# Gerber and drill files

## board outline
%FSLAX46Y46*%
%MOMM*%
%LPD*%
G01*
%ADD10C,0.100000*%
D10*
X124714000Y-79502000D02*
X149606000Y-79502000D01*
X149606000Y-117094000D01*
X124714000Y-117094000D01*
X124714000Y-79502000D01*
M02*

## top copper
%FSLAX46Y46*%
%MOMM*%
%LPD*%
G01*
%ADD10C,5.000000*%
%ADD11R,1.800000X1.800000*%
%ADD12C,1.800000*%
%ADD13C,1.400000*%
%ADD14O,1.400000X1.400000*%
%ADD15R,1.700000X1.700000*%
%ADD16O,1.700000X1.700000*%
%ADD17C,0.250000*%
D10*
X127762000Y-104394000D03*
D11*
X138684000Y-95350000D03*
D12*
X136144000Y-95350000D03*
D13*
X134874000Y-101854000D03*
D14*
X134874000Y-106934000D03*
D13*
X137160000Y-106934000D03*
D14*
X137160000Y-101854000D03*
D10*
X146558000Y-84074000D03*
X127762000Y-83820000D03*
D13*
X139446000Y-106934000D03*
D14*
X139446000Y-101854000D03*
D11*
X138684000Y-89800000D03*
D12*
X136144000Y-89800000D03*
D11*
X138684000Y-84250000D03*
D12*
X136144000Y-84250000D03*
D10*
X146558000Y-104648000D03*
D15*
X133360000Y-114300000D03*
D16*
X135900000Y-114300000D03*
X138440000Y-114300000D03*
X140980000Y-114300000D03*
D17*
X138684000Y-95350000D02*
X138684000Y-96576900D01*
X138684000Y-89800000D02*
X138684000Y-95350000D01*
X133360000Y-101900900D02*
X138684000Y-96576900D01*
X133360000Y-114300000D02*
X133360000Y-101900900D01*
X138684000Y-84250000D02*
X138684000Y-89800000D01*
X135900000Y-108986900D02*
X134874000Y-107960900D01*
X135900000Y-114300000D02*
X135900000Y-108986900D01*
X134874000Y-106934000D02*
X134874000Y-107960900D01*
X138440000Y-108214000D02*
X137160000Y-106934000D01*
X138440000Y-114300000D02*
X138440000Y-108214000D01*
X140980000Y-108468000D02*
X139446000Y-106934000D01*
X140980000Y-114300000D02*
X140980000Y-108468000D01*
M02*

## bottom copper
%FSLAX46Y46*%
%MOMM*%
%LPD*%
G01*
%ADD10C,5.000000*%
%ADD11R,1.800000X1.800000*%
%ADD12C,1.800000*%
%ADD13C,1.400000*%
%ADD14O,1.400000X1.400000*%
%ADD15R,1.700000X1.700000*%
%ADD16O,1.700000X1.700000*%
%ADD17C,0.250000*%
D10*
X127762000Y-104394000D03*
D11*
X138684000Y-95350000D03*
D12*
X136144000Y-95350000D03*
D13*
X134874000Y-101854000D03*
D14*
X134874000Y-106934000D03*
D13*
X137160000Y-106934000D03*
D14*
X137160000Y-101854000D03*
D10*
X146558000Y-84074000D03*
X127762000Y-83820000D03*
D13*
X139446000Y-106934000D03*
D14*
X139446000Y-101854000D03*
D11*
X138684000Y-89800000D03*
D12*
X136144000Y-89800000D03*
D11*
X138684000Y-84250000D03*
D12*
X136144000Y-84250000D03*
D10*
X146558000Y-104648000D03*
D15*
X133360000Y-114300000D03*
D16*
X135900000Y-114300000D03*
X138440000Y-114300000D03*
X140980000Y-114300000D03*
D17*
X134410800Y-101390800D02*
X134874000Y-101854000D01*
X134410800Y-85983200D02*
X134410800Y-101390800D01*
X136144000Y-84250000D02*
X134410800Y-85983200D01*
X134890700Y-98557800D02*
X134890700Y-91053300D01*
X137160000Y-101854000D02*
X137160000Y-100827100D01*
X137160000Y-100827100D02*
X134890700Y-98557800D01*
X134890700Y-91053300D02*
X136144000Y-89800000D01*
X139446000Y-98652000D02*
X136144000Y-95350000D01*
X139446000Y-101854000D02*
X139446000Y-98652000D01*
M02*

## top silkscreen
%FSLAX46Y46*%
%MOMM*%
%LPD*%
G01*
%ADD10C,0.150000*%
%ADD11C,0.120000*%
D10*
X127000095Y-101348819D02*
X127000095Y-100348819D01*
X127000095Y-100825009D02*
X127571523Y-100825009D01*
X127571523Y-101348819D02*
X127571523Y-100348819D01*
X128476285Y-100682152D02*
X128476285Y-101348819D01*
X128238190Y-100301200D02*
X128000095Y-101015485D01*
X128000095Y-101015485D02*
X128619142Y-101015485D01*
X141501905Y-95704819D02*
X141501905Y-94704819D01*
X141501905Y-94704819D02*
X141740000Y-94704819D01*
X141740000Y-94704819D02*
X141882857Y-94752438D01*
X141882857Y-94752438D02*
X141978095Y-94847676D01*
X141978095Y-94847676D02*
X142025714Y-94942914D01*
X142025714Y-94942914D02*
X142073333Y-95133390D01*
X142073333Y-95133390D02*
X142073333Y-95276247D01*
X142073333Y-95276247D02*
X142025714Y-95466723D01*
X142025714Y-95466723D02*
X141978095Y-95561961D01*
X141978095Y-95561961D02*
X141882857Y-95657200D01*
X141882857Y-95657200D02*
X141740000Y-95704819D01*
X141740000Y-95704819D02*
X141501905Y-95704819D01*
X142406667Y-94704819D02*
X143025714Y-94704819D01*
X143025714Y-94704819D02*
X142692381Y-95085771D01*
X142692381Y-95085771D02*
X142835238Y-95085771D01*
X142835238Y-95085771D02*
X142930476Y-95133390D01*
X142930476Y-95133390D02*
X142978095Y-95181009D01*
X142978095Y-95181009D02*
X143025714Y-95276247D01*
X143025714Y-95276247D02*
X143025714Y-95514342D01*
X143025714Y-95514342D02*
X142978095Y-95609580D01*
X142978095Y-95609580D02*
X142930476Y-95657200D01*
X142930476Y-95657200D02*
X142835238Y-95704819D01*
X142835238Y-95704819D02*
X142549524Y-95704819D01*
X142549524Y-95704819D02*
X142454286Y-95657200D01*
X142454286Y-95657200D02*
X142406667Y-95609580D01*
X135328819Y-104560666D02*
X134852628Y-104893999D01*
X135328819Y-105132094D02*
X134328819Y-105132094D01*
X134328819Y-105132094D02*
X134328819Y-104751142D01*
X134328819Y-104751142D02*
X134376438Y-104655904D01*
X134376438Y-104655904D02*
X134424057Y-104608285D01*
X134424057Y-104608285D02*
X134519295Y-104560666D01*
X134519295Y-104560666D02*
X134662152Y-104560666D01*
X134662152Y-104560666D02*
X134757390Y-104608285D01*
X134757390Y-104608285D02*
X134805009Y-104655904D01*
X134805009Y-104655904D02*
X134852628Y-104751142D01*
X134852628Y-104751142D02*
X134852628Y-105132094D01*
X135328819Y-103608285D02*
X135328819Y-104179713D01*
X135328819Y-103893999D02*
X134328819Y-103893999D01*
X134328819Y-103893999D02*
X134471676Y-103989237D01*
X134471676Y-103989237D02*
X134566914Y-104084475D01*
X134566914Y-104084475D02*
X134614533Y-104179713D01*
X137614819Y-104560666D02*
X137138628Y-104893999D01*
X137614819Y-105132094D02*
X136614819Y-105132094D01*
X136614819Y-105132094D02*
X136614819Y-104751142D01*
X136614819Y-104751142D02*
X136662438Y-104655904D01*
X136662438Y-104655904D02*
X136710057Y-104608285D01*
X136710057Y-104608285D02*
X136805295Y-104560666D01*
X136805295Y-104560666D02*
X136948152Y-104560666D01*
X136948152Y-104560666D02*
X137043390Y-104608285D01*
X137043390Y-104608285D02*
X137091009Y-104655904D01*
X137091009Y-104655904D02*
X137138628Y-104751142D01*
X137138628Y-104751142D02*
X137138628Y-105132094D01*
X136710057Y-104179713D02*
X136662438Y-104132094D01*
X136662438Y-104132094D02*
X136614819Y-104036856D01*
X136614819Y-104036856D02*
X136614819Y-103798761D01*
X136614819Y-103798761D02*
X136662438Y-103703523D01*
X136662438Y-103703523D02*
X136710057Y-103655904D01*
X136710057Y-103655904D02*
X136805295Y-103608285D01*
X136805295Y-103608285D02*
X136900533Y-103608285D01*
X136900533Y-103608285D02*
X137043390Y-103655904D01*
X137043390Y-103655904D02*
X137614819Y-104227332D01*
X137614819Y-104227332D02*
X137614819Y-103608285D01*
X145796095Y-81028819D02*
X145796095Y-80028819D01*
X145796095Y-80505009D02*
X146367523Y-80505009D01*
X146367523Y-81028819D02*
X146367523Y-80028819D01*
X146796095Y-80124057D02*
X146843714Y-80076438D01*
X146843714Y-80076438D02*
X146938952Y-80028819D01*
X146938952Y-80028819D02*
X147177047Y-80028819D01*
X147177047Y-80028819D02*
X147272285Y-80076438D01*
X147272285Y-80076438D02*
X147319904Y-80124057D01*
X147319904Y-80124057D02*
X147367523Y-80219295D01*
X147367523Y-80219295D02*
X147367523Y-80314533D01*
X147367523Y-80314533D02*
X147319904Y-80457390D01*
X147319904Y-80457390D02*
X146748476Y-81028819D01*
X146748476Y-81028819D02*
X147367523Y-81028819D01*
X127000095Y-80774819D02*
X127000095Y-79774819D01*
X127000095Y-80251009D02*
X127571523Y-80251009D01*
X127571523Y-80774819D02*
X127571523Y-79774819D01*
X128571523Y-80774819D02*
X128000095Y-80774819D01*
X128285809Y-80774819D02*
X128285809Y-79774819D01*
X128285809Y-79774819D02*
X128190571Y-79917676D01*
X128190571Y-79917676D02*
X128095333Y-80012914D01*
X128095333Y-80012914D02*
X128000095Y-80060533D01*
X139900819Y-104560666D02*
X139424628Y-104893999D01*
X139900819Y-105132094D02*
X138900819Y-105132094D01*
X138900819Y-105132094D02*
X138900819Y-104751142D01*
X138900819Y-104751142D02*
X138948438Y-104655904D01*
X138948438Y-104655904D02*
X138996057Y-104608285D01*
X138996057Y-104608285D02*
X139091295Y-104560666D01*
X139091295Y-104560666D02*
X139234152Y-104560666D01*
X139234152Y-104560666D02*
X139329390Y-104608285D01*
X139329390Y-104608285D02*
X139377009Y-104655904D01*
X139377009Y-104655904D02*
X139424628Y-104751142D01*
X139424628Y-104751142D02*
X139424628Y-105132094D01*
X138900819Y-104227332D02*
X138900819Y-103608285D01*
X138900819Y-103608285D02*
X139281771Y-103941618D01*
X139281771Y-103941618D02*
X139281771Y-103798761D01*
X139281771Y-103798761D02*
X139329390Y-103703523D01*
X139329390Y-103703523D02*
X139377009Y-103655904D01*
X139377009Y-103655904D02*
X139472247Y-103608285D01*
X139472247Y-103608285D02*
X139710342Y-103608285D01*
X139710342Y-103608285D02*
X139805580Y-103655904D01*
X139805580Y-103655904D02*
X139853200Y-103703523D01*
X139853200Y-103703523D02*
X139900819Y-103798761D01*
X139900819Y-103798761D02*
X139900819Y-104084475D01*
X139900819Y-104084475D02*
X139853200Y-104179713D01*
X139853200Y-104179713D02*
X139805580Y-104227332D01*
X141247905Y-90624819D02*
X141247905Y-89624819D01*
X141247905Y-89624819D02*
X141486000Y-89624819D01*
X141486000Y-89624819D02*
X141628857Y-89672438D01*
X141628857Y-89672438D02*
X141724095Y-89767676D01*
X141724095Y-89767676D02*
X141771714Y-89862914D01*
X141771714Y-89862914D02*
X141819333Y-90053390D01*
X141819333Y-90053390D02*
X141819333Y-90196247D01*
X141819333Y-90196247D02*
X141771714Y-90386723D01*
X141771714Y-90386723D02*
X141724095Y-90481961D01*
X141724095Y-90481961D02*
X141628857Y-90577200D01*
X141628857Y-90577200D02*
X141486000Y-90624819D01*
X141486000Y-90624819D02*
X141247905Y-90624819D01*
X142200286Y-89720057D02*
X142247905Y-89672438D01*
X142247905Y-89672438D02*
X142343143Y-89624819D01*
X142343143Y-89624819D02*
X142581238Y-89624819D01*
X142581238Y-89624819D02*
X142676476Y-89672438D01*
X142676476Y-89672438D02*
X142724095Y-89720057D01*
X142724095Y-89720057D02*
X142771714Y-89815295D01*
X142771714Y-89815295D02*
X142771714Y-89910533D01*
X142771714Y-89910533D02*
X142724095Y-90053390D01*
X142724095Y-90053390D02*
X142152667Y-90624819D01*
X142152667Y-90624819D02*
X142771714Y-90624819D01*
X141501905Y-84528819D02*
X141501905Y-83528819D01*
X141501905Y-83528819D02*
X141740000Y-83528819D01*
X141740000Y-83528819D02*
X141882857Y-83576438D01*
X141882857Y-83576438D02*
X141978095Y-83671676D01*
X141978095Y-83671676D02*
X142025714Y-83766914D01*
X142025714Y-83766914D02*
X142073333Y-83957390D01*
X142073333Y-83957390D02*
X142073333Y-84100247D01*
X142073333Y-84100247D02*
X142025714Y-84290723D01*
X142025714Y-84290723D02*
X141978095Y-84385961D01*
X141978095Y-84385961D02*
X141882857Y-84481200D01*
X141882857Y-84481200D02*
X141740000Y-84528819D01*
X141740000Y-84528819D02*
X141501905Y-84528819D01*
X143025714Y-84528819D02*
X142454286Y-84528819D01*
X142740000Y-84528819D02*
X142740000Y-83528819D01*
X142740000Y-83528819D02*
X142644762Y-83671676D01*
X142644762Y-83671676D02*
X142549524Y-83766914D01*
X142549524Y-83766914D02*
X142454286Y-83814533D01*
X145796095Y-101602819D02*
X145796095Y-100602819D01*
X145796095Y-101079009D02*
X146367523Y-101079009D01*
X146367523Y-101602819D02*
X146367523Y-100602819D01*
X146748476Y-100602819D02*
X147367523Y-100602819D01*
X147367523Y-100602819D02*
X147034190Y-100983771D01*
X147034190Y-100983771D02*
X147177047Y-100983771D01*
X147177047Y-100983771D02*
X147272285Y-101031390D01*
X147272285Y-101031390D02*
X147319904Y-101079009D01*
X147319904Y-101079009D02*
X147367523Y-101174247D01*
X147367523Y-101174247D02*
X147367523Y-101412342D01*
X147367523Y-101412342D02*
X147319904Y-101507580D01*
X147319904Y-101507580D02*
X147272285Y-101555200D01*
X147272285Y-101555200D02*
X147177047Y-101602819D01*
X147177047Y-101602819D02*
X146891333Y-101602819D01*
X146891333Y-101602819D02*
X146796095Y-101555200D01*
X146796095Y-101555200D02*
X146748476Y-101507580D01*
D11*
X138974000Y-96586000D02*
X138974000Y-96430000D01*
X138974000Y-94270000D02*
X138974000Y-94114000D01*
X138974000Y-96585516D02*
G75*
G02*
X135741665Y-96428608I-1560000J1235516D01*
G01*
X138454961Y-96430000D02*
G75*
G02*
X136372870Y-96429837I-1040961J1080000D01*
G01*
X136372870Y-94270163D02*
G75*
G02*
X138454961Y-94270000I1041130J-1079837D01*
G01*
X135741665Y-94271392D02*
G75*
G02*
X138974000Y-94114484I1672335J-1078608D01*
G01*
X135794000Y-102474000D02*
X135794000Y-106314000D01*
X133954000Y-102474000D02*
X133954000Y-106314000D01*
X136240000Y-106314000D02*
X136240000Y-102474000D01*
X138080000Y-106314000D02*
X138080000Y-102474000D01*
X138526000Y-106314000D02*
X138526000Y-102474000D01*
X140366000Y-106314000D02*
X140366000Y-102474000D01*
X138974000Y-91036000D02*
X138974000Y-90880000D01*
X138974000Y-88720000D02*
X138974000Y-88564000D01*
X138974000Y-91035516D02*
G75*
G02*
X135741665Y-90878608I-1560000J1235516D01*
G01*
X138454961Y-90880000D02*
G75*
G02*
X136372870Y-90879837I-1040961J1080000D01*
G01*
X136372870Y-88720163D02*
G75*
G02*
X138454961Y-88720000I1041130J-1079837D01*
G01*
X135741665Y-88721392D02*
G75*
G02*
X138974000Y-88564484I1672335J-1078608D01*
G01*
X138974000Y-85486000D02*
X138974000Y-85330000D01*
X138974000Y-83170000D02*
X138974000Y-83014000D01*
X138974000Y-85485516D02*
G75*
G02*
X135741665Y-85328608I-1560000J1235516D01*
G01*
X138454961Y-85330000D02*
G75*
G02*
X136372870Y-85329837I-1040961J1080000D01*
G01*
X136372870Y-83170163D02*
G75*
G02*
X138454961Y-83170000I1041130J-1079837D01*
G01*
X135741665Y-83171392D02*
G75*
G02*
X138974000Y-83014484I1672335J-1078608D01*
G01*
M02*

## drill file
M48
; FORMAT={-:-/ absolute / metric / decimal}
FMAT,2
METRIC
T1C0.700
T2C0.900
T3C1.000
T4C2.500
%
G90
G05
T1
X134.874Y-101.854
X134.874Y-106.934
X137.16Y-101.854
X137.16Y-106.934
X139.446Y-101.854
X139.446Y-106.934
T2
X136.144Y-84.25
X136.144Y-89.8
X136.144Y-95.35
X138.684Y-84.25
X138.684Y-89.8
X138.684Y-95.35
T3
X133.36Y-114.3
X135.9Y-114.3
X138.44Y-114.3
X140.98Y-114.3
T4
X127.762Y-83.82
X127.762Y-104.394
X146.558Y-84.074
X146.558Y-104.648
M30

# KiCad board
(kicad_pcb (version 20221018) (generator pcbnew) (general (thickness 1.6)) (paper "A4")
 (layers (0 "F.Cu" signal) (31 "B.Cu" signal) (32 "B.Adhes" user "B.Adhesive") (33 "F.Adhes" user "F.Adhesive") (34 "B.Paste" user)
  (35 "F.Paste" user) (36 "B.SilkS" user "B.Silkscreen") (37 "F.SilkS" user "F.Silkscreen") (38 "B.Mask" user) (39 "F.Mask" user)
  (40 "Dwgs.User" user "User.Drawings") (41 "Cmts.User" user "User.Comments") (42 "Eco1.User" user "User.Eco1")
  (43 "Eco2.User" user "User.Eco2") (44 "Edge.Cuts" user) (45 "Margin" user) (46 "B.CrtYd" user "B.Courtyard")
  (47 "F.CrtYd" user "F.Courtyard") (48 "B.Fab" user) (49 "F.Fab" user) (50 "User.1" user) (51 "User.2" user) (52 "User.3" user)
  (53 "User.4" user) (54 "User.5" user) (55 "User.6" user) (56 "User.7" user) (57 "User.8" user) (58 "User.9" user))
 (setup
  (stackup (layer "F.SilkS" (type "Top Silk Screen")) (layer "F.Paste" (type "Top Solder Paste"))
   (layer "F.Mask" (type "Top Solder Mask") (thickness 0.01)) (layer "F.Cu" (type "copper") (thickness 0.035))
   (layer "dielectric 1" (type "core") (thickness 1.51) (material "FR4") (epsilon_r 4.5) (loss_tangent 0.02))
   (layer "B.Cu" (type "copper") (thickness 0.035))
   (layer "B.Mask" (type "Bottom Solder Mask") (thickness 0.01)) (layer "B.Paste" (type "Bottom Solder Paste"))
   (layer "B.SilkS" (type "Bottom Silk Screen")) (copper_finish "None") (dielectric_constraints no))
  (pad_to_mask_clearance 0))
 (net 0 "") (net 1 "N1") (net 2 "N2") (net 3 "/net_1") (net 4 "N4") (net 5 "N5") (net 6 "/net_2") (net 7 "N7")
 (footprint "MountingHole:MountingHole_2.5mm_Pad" (layer "F.Cu") (at 127.762 104.394)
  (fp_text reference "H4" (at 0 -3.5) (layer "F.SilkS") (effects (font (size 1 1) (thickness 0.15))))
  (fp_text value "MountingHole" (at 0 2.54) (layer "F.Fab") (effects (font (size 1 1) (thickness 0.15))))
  (pad "1" thru_hole circle (at 0 0) (size 5 5) (drill 2.5) (layers "*.Cu" "*.Mask")))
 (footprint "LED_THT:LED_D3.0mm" (layer "F.Cu") (at 138.684 95.35 180)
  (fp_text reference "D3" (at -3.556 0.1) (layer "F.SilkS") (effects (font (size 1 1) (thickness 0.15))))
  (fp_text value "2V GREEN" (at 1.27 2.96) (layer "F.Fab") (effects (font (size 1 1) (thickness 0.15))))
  (fp_line (start -0.29 -1.236) (end -0.29 -1.08) (stroke (width 0.12) (type solid)) (layer "F.SilkS"))
  (fp_line (start -0.29 1.08) (end -0.29 1.236) (stroke (width 0.12) (type solid)) (layer "F.SilkS"))
  (fp_arc (start -0.29 -1.235516) (mid 1.366487 -1.987659) (end 2.942335 -1.078608) (stroke (width 0.12) (type solid)) (layer "F.SilkS"))
  (fp_arc (start 0.229039 -1.08) (mid 1.270117 -1.5) (end 2.31113 -1.079837) (stroke (width 0.12) (type solid)) (layer "F.SilkS"))
  (fp_arc (start 2.31113 1.079837) (mid 1.270117 1.5) (end 0.229039 1.08) (stroke (width 0.12) (type solid)) (layer "F.SilkS"))
  (fp_arc (start 2.942335 1.078608) (mid 1.366487 1.987659) (end -0.29 1.235516) (stroke (width 0.12) (type solid)) (layer "F.SilkS"))
  (pad "1" thru_hole rect (at 0 0 180) (size 1.8 1.8) (drill 0.9) (layers "*.Cu" "*.Mask") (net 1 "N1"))
  (pad "2" thru_hole circle (at 2.54 0 180) (size 1.8 1.8) (drill 0.9) (layers "*.Cu" "*.Mask") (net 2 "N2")))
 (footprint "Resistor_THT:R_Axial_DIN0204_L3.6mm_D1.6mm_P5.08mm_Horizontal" (layer "F.Cu") (at 134.874 101.854 -90)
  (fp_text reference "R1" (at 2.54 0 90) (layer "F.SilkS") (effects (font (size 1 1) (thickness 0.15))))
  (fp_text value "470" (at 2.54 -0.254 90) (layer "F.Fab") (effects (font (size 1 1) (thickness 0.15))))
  (fp_line (start 0.62 -0.92) (end 4.46 -0.92) (stroke (width 0.12) (type solid)) (layer "F.SilkS"))
  (fp_line (start 0.62 0.92) (end 4.46 0.92) (stroke (width 0.12) (type solid)) (layer "F.SilkS"))
  (pad "1" thru_hole circle (at 0 0 270) (size 1.4 1.4) (drill 0.7) (layers "*.Cu" "*.Mask") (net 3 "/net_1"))
  (pad "2" thru_hole oval (at 5.08 0 270) (size 1.4 1.4) (drill 0.7) (layers "*.Cu" "*.Mask") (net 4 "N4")))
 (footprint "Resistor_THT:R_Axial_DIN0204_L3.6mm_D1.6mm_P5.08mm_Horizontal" (layer "F.Cu") (at 137.16 106.934 90)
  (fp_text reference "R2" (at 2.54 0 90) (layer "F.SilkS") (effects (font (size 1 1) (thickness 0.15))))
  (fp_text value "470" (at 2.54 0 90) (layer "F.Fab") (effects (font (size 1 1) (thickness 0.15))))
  (fp_line (start 0.62 -0.92) (end 4.46 -0.92) (stroke (width 0.12) (type solid)) (layer "F.SilkS"))
  (fp_line (start 0.62 0.92) (end 4.46 0.92) (stroke (width 0.12) (type solid)) (layer "F.SilkS"))
  (pad "1" thru_hole circle (at 0 0 90) (size 1.4 1.4) (drill 0.7) (layers "*.Cu" "*.Mask") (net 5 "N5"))
  (pad "2" thru_hole oval (at 5.08 0 90) (size 1.4 1.4) (drill 0.7) (layers "*.Cu" "*.Mask") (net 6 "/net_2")))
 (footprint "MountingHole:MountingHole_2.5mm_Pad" (layer "F.Cu") (at 146.558 84.074)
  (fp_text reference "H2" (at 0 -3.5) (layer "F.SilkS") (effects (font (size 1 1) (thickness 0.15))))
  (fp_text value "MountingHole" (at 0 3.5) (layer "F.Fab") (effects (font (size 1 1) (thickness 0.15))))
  (pad "1" thru_hole circle (at 0 0) (size 5 5) (drill 2.5) (layers "*.Cu" "*.Mask")))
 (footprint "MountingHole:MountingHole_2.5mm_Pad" (layer "F.Cu") (at 127.762 83.82)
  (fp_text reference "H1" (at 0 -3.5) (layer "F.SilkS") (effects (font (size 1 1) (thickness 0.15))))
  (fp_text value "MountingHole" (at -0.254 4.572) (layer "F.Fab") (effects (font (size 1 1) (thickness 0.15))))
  (pad "1" thru_hole circle (at 0 0) (size 5 5) (drill 2.5) (layers "*.Cu" "*.Mask")))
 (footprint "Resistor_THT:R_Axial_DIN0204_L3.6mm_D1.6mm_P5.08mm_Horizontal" (layer "F.Cu") (at 139.446 106.934 90)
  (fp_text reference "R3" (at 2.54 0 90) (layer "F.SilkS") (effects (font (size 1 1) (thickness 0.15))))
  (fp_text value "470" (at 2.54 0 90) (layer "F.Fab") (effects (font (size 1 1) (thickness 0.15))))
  (fp_line (start 0.62 -0.92) (end 4.46 -0.92) (stroke (width 0.12) (type solid)) (layer "F.SilkS"))
  (fp_line (start 0.62 0.92) (end 4.46 0.92) (stroke (width 0.12) (type solid)) (layer "F.SilkS"))
  (pad "1" thru_hole circle (at 0 0 90) (size 1.4 1.4) (drill 0.7) (layers "*.Cu" "*.Mask") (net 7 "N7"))
  (pad "2" thru_hole oval (at 5.08 0 90) (size 1.4 1.4) (drill 0.7) (layers "*.Cu" "*.Mask") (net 2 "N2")))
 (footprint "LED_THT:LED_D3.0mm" (layer "F.Cu") (at 138.684 89.8 180)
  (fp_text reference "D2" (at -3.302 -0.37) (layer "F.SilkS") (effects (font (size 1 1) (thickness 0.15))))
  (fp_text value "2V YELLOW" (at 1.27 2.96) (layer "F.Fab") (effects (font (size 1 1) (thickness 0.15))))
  (fp_line (start -0.29 -1.236) (end -0.29 -1.08) (stroke (width 0.12) (type solid)) (layer "F.SilkS"))
  (fp_line (start -0.29 1.08) (end -0.29 1.236) (stroke (width 0.12) (type solid)) (layer "F.SilkS"))
  (fp_arc (start -0.29 -1.235516) (mid 1.366487 -1.987659) (end 2.942335 -1.078608) (stroke (width 0.12) (type solid)) (layer "F.SilkS"))
  (fp_arc (start 0.229039 -1.08) (mid 1.270117 -1.5) (end 2.31113 -1.079837) (stroke (width 0.12) (type solid)) (layer "F.SilkS"))
  (fp_arc (start 2.31113 1.079837) (mid 1.270117 1.5) (end 0.229039 1.08) (stroke (width 0.12) (type solid)) (layer "F.SilkS"))
  (fp_arc (start 2.942335 1.078608) (mid 1.366487 1.987659) (end -0.29 1.235516) (stroke (width 0.12) (type solid)) (layer "F.SilkS"))
  (pad "1" thru_hole rect (at 0 0 180) (size 1.8 1.8) (drill 0.9) (layers "*.Cu" "*.Mask") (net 1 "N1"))
  (pad "2" thru_hole circle (at 2.54 0 180) (size 1.8 1.8) (drill 0.9) (layers "*.Cu" "*.Mask") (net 6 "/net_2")))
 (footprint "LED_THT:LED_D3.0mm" (layer "F.Cu") (at 138.684 84.25 180)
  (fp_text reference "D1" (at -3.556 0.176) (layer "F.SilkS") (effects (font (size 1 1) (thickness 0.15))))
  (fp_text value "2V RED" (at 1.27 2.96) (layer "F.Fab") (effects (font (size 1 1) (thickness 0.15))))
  (fp_line (start -0.29 -1.236) (end -0.29 -1.08) (stroke (width 0.12) (type solid)) (layer "F.SilkS"))
  (fp_line (start -0.29 1.08) (end -0.29 1.236) (stroke (width 0.12) (type solid)) (layer "F.SilkS"))
  (fp_arc (start -0.29 -1.235516) (mid 1.366487 -1.987659) (end 2.942335 -1.078608) (stroke (width 0.12) (type solid)) (layer "F.SilkS"))
  (fp_arc (start 0.229039 -1.08) (mid 1.270117 -1.5) (end 2.31113 -1.079837) (stroke (width 0.12) (type solid)) (layer "F.SilkS"))
  (fp_arc (start 2.31113 1.079837) (mid 1.270117 1.5) (end 0.229039 1.08) (stroke (width 0.12) (type solid)) (layer "F.SilkS"))
  (fp_arc (start 2.942335 1.078608) (mid 1.366487 1.987659) (end -0.29 1.235516) (stroke (width 0.12) (type solid)) (layer "F.SilkS"))
  (pad "1" thru_hole rect (at 0 0 180) (size 1.8 1.8) (drill 0.9) (layers "*.Cu" "*.Mask") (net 1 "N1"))
  (pad "2" thru_hole circle (at 2.54 0 180) (size 1.8 1.8) (drill 0.9) (layers "*.Cu" "*.Mask") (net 3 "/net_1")))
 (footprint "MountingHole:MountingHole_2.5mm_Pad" (layer "F.Cu") (at 146.558 104.648)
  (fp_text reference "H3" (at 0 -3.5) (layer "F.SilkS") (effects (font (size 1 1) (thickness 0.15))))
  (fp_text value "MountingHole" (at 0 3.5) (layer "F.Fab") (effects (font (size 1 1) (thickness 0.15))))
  (pad "1" thru_hole circle (at 0 0) (size 5 5) (drill 2.5) (layers "*.Cu" "*.Mask")))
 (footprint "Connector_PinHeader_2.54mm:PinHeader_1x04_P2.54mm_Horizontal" (layer "B.Cu") (at 133.36 114.3 -90)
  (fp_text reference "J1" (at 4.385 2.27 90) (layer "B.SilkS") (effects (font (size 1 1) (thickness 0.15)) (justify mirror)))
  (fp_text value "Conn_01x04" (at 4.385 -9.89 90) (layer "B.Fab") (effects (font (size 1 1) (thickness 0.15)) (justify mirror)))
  (pad "1" thru_hole rect (at 0 0 270) (size 1.7 1.7) (drill 1) (layers "*.Cu" "*.Mask") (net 1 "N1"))
  (pad "2" thru_hole oval (at 0 -2.54 270) (size 1.7 1.7) (drill 1) (layers "*.Cu" "*.Mask") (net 4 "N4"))
  (pad "3" thru_hole oval (at 0 -5.08 270) (size 1.7 1.7) (drill 1) (layers "*.Cu" "*.Mask") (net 5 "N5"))
  (pad "4" thru_hole oval (at 0 -7.62 270) (size 1.7 1.7) (drill 1) (layers "*.Cu" "*.Mask") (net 7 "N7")))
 (gr_rect (start 124.714 79.502) (end 149.606 117.094) (stroke (width 0.1) (type default)) (fill none) (layer "Edge.Cuts"))
 (segment (start 138.684 95.35) (end 138.684 96.5769) (width 0.25) (layer "F.Cu") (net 1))
 (segment (start 138.684 89.8) (end 138.684 95.35) (width 0.25) (layer "F.Cu") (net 1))
 (segment (start 133.36 101.9009) (end 138.684 96.5769) (width 0.25) (layer "F.Cu") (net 1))
 (segment (start 133.36 114.3) (end 133.36 101.9009) (width 0.25) (layer "F.Cu") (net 1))
 (segment (start 138.684 84.25) (end 138.684 89.8) (width 0.25) (layer "F.Cu") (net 1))
 (segment (start 134.4108 101.3908) (end 134.874 101.854) (width 0.25) (layer "B.Cu") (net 3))
 (segment (start 134.4108 85.9832) (end 134.4108 101.3908) (width 0.25) (layer "B.Cu") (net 3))
 (segment (start 136.144 84.25) (end 134.4108 85.9832) (width 0.25) (layer "B.Cu") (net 3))
 (segment (start 134.8907 98.5578) (end 134.8907 91.0533) (width 0.25) (layer "B.Cu") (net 6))
 (segment (start 137.16 101.854) (end 137.16 100.8271) (width 0.25) (layer "B.Cu") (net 6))
 (segment (start 137.16 100.8271) (end 134.8907 98.5578) (width 0.25) (layer "B.Cu") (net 6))
 (segment (start 134.8907 91.0533) (end 136.144 89.8) (width 0.25) (layer "B.Cu") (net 6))
 (segment (start 139.446 98.652) (end 136.144 95.35) (width 0.25) (layer "B.Cu") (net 2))
 (segment (start 139.446 101.854) (end 139.446 98.652) (width 0.25) (layer "B.Cu") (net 2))
 (segment (start 135.9 108.9869) (end 134.874 107.9609) (width 0.25) (layer "F.Cu") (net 4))
 (segment (start 135.9 114.3) (end 135.9 108.9869) (width 0.25) (layer "F.Cu") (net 4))
 (segment (start 134.874 106.934) (end 134.874 107.9609) (width 0.25) (layer "F.Cu") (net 4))
 (segment (start 138.44 108.214) (end 137.16 106.934) (width 0.25) (layer "F.Cu") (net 5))
 (segment (start 138.44 114.3) (end 138.44 108.214) (width 0.25) (layer "F.Cu") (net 5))
 (segment (start 140.98 108.468) (end 139.446 106.934) (width 0.25) (layer "F.Cu") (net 7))
 (segment (start 140.98 114.3) (end 140.98 108.468) (width 0.25) (layer "F.Cu") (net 7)))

